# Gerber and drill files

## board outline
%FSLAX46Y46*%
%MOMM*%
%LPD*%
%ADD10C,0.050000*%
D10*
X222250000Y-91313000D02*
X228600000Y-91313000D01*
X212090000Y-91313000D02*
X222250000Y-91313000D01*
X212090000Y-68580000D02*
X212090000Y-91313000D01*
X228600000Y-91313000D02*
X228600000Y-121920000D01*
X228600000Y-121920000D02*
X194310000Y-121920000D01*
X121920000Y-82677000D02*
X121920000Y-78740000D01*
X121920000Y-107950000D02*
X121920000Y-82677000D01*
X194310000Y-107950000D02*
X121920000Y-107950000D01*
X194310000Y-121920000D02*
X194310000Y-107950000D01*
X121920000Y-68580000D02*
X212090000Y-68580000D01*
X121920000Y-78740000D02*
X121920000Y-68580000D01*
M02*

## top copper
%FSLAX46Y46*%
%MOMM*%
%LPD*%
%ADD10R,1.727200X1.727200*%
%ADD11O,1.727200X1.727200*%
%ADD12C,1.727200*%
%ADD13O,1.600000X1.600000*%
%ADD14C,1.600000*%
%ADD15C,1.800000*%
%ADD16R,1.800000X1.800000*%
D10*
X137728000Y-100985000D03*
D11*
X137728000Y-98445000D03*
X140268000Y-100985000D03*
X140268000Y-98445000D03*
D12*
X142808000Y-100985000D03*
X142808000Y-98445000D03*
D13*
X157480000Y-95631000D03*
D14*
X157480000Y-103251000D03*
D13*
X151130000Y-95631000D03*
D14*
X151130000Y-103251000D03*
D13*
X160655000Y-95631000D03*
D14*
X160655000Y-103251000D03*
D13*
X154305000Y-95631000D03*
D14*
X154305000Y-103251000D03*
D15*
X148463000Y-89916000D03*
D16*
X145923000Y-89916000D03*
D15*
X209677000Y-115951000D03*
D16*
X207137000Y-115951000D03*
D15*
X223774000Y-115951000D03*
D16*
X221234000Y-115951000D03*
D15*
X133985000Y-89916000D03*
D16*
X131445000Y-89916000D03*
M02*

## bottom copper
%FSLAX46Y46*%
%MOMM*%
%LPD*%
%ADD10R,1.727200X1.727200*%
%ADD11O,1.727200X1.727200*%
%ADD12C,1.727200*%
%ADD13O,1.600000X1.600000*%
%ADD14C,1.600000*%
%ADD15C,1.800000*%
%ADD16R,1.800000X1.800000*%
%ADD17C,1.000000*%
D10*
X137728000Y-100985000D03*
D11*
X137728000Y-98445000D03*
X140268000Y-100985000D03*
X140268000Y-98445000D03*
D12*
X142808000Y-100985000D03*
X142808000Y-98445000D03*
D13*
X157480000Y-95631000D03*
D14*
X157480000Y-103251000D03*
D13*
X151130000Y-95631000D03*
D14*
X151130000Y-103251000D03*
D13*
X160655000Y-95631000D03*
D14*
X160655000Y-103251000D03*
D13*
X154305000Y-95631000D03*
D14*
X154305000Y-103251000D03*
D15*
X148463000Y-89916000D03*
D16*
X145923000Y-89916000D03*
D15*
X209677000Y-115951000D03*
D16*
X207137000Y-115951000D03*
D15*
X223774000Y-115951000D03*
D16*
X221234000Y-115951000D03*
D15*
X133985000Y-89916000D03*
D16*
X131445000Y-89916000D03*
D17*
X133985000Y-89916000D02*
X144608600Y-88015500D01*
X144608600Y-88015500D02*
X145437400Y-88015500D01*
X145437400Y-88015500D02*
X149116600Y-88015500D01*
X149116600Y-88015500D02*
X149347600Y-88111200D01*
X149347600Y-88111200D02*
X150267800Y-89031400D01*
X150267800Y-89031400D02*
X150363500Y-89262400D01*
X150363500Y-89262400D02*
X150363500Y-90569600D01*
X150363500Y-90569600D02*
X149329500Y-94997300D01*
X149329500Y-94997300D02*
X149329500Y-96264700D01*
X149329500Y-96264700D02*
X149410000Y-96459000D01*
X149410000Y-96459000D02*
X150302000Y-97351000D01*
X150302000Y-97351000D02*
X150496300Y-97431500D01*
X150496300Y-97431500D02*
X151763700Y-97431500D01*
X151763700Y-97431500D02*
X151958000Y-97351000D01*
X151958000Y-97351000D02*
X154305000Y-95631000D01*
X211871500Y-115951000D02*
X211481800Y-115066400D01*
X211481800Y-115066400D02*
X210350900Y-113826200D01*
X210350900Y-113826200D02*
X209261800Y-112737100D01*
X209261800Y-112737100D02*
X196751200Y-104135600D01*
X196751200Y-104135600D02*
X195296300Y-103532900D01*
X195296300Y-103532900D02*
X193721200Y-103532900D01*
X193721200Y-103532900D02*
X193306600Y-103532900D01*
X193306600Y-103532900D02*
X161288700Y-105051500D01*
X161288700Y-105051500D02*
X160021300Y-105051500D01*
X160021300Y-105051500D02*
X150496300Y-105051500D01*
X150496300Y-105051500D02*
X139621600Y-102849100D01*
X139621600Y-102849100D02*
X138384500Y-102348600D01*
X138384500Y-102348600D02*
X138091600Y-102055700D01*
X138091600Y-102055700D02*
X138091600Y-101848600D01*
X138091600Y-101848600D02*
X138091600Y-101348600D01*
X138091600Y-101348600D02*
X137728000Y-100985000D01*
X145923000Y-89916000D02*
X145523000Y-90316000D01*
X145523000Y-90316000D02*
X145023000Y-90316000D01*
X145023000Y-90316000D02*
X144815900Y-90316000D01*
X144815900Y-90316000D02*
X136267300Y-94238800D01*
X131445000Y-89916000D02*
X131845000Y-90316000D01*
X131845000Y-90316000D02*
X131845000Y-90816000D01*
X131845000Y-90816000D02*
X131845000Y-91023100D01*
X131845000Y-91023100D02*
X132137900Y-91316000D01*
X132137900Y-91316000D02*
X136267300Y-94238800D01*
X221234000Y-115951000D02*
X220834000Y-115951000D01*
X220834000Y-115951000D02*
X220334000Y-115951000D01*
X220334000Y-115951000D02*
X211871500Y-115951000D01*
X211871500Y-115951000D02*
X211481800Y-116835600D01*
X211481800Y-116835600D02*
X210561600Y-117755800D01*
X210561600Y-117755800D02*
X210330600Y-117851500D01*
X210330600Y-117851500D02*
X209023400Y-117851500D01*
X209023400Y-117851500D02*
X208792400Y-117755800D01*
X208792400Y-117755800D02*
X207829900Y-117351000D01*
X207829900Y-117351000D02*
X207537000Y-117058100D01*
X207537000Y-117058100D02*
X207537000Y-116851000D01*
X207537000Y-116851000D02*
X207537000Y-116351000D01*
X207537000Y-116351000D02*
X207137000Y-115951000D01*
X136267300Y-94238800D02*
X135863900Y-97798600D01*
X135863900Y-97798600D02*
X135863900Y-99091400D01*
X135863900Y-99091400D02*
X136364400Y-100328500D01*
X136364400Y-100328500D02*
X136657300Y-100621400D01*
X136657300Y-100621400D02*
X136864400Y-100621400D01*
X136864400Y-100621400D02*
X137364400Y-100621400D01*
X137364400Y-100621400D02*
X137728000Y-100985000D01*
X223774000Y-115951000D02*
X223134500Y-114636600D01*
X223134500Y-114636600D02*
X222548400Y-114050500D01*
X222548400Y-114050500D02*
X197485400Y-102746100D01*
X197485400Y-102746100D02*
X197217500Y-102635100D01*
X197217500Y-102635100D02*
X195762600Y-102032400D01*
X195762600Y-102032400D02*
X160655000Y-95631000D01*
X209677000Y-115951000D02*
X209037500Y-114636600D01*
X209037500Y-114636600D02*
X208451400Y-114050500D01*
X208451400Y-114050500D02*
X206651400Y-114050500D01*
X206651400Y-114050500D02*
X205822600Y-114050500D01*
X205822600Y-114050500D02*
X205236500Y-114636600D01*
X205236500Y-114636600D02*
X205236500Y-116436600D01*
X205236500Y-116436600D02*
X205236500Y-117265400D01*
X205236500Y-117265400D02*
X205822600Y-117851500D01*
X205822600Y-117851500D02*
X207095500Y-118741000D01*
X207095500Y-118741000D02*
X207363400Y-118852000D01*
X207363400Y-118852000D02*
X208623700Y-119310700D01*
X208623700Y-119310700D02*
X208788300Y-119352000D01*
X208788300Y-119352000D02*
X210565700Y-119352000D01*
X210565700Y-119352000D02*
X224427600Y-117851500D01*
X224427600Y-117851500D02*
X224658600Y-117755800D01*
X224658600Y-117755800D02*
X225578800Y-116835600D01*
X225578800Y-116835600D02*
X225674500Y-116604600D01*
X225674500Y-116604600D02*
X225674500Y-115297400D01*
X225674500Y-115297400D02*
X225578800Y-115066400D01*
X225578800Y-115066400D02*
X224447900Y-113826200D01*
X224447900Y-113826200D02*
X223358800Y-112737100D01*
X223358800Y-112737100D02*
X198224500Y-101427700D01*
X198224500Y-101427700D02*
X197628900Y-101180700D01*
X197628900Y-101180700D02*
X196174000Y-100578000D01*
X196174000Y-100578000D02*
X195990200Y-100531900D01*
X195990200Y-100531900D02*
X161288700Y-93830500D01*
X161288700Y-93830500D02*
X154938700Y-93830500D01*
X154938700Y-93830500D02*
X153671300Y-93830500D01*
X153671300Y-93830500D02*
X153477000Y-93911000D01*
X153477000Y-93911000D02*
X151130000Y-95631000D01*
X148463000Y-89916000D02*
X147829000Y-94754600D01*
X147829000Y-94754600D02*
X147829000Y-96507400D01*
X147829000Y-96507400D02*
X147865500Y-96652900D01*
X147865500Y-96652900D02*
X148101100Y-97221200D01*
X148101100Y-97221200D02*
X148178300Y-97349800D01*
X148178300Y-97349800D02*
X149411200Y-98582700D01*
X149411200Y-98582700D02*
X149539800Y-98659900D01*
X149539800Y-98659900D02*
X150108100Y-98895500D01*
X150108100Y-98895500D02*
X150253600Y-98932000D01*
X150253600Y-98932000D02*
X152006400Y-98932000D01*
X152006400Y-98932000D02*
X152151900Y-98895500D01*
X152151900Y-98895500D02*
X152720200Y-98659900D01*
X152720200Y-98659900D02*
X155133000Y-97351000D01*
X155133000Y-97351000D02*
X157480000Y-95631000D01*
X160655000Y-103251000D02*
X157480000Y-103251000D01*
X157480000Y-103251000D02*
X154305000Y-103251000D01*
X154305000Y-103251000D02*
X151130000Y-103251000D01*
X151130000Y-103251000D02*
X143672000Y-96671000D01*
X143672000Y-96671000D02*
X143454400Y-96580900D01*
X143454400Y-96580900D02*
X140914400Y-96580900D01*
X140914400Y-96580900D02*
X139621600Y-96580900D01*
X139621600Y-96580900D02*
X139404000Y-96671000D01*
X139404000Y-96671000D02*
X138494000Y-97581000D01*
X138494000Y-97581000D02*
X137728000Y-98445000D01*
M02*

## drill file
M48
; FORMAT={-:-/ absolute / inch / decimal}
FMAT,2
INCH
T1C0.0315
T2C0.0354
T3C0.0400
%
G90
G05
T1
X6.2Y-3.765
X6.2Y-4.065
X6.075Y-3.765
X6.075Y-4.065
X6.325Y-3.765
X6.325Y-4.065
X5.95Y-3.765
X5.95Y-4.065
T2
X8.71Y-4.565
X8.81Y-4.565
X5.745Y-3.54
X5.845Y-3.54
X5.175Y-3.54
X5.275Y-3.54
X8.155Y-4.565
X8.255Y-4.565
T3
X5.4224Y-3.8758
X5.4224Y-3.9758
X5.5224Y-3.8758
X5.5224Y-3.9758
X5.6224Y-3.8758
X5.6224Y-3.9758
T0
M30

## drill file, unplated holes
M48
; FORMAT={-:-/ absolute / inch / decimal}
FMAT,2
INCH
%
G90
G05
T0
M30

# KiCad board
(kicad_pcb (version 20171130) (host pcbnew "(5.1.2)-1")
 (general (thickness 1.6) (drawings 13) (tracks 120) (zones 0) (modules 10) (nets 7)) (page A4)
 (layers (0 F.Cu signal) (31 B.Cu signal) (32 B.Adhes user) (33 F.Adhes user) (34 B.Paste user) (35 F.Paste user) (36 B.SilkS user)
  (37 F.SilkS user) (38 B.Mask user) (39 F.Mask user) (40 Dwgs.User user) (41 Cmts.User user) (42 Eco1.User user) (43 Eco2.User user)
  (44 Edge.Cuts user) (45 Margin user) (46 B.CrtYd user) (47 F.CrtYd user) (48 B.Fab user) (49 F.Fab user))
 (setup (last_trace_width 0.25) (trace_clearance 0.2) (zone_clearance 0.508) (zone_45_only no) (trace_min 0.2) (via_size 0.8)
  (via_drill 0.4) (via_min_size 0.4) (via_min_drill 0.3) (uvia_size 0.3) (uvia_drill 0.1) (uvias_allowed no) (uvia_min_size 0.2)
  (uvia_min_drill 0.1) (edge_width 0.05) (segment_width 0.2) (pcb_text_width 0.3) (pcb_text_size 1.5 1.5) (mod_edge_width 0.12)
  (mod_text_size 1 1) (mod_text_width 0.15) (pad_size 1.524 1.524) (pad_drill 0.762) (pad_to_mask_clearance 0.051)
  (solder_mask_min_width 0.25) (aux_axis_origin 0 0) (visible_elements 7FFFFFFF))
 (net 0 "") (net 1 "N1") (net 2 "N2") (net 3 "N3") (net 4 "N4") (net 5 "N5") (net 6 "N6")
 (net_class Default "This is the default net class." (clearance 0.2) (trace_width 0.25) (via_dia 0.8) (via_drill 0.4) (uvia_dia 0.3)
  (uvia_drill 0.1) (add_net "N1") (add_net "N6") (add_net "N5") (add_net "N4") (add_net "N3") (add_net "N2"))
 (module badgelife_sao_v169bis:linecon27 (layer F.Cu) (at 173.482 93.345)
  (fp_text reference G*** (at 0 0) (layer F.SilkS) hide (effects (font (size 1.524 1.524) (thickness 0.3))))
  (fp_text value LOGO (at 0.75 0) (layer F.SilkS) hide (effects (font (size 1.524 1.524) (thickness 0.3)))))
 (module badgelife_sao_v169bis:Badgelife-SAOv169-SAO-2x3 (layer F.Cu) (at 140.208 99.695)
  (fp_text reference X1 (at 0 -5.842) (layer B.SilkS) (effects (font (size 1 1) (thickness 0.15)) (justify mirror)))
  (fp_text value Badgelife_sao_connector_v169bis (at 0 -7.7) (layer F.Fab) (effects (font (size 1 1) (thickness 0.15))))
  (pad 2 thru_hole rect (at -2.48 1.29 270) (size 1.7272 1.7272) (drill 1.016) (layers *.Cu *.Mask) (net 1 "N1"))
  (pad 1 thru_hole oval (at -2.48 -1.25 270) (size 1.7272 1.7272) (drill 1.016) (layers *.Cu *.Mask) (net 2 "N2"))
  (pad 4 thru_hole oval (at 0.06 1.29 270) (size 1.7272 1.7272) (drill 1.016) (layers *.Cu *.Mask))
  (pad 3 thru_hole oval (at 0.06 -1.25 270) (size 1.7272 1.7272) (drill 1.016) (layers *.Cu *.Mask))
  (pad 6 thru_hole circle (at 2.6 1.29 270) (size 1.7272 1.7272) (drill 1.016) (layers *.Cu *.Mask))
  (pad 5 thru_hole circle (at 2.6 -1.25 270) (size 1.7272 1.7272) (drill 1.016) (layers *.Cu *.Mask)))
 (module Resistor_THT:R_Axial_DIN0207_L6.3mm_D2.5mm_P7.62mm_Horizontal (layer F.Cu) (at 157.48 103.251 90)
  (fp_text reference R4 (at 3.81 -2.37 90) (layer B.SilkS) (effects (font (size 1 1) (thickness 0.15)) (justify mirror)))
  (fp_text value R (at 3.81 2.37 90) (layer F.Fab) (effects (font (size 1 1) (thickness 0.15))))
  (pad 2 thru_hole oval (at 7.62 0 90) (size 1.6 1.6) (drill 0.8) (layers *.Cu *.Mask) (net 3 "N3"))
  (pad 1 thru_hole circle (at 0 0 90) (size 1.6 1.6) (drill 0.8) (layers *.Cu *.Mask) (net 2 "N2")))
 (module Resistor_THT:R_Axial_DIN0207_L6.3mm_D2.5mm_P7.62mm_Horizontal (layer F.Cu) (at 151.13 103.251 90)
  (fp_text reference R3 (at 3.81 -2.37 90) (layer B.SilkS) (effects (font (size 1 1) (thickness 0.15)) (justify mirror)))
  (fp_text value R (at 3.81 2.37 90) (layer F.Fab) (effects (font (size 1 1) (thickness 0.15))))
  (pad 2 thru_hole oval (at 7.62 0 90) (size 1.6 1.6) (drill 0.8) (layers *.Cu *.Mask) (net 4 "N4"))
  (pad 1 thru_hole circle (at 0 0 90) (size 1.6 1.6) (drill 0.8) (layers *.Cu *.Mask) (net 2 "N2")))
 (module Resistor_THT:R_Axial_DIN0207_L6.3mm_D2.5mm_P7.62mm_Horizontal (layer F.Cu) (at 160.655 103.251 90)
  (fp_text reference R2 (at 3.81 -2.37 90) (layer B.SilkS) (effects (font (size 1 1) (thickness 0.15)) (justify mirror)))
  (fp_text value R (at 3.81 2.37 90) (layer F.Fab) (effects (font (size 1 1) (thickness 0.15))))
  (pad 2 thru_hole oval (at 7.62 0 90) (size 1.6 1.6) (drill 0.8) (layers *.Cu *.Mask) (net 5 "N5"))
  (pad 1 thru_hole circle (at 0 0 90) (size 1.6 1.6) (drill 0.8) (layers *.Cu *.Mask) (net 2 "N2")))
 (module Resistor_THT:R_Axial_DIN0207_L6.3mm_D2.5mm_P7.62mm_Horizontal (layer F.Cu) (at 154.305 103.251 90)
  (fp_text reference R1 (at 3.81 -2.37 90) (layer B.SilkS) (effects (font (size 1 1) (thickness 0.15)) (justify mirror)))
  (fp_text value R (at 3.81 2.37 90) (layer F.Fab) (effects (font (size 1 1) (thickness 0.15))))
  (pad 2 thru_hole oval (at 7.62 0 90) (size 1.6 1.6) (drill 0.8) (layers *.Cu *.Mask) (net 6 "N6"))
  (pad 1 thru_hole circle (at 0 0 90) (size 1.6 1.6) (drill 0.8) (layers *.Cu *.Mask) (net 2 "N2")))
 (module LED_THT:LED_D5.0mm (layer F.Cu) (at 145.923 89.916)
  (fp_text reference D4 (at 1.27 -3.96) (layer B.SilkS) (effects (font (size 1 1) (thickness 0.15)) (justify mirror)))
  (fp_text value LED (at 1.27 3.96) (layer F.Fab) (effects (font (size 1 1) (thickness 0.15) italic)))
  (pad 2 thru_hole circle (at 2.54 0) (size 1.8 1.8) (drill 0.9) (layers *.Cu *.Mask) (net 3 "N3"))
  (pad 1 thru_hole rect (at 0 0) (size 1.8 1.8) (drill 0.9) (layers *.Cu *.Mask) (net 1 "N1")))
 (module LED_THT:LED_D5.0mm (layer F.Cu) (at 207.137 115.951)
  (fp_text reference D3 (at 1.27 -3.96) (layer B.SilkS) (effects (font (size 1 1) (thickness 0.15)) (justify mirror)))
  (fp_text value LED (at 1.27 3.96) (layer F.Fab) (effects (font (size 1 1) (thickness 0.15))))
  (pad 2 thru_hole circle (at 2.54 0) (size 1.8 1.8) (drill 0.9) (layers *.Cu *.Mask) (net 4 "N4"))
  (pad 1 thru_hole rect (at 0 0) (size 1.8 1.8) (drill 0.9) (layers *.Cu *.Mask) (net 1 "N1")))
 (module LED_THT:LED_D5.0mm (layer F.Cu) (at 221.234 115.951)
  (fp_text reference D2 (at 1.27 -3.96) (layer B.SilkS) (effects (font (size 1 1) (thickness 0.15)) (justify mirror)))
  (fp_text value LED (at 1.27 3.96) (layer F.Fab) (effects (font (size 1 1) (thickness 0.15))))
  (pad 2 thru_hole circle (at 2.54 0) (size 1.8 1.8) (drill 0.9) (layers *.Cu *.Mask) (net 5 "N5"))
  (pad 1 thru_hole rect (at 0 0) (size 1.8 1.8) (drill 0.9) (layers *.Cu *.Mask) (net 1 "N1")))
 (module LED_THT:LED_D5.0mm (layer F.Cu) (at 131.445 89.916)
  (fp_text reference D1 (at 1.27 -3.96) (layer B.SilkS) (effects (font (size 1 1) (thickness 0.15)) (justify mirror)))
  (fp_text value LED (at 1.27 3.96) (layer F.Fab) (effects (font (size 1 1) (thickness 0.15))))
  (pad 2 thru_hole circle (at 2.54 0) (size 1.8 1.8) (drill 0.9) (layers *.Cu *.Mask) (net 6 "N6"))
  (pad 1 thru_hole rect (at 0 0) (size 1.8 1.8) (drill 0.9) (layers *.Cu *.Mask) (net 1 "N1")))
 (gr_line (start 222.25 91.313) (end 228.6 91.313) (layer Edge.Cuts) (width 0.05))
 (gr_line (start 212.09 91.313) (end 222.25 91.313) (layer Edge.Cuts) (width 0.05))
 (gr_line (start 212.09 68.58) (end 212.09 91.313) (layer Edge.Cuts) (width 0.05))
 (gr_line (start 228.6 91.313) (end 228.6 121.92) (layer Edge.Cuts) (width 0.05))
 (gr_line (start 228.6 121.92) (end 194.31 121.92) (layer Edge.Cuts) (width 0.05))
 (gr_line (start 121.92 82.677) (end 121.92 78.74) (layer Edge.Cuts) (width 0.05))
 (gr_line (start 121.92 107.95) (end 121.92 82.677) (layer Edge.Cuts) (width 0.05))
 (gr_line (start 194.31 107.95) (end 121.92 107.95) (layer Edge.Cuts) (width 0.05))
 (gr_line (start 194.31 121.92) (end 194.31 107.95) (layer Edge.Cuts) (width 0.05))
 (gr_line (start 121.92 68.58) (end 212.09 68.58) (layer Edge.Cuts) (width 0.05))
 (gr_line (start 121.92 78.74) (end 121.92 68.58) (layer Edge.Cuts) (width 0.05))
 (segment (start 133.985 89.916) (end 144.6086 88.0155) (width 1) (layer B.Cu) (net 6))
 (segment (start 144.6086 88.0155) (end 145.4374 88.0155) (width 1) (layer B.Cu) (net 6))
 (segment (start 145.4374 88.0155) (end 149.1166 88.0155) (width 1) (layer B.Cu) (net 6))
 (segment (start 149.1166 88.0155) (end 149.3476 88.1112) (width 1) (layer B.Cu) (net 6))
 (segment (start 149.3476 88.1112) (end 150.2678 89.0314) (width 1) (layer B.Cu) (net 6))
 (segment (start 150.2678 89.0314) (end 150.3635 89.2624) (width 1) (layer B.Cu) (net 6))
 (segment (start 150.3635 89.2624) (end 150.3635 90.5696) (width 1) (layer B.Cu) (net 6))
 (segment (start 150.3635 90.5696) (end 149.3295 94.9973) (width 1) (layer B.Cu) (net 6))
 (segment (start 149.3295 94.9973) (end 149.3295 96.2647) (width 1) (layer B.Cu) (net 6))
 (segment (start 149.3295 96.2647) (end 149.41 96.459) (width 1) (layer B.Cu) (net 6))
 (segment (start 149.41 96.459) (end 150.302 97.351) (width 1) (layer B.Cu) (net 6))
 (segment (start 150.302 97.351) (end 150.4963 97.4315) (width 1) (layer B.Cu) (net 6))
 (segment (start 150.4963 97.4315) (end 151.7637 97.4315) (width 1) (layer B.Cu) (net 6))
 (segment (start 151.7637 97.4315) (end 151.958 97.351) (width 1) (layer B.Cu) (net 6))
 (segment (start 151.958 97.351) (end 154.305 95.631) (width 1) (layer B.Cu) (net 6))
 (segment (start 211.8715 115.951) (end 211.4818 115.0664) (width 1) (layer B.Cu) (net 1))
 (segment (start 211.4818 115.0664) (end 210.3509 113.8262) (width 1) (layer B.Cu) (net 1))
 (segment (start 210.3509 113.8262) (end 209.2618 112.7371) (width 1) (layer B.Cu) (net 1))
 (segment (start 209.2618 112.7371) (end 196.7512 104.1356) (width 1) (layer B.Cu) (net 1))
 (segment (start 196.7512 104.1356) (end 195.2963 103.5329) (width 1) (layer B.Cu) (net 1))
 (segment (start 195.2963 103.5329) (end 193.7212 103.5329) (width 1) (layer B.Cu) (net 1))
 (segment (start 193.7212 103.5329) (end 193.3066 103.5329) (width 1) (layer B.Cu) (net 1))
 (segment (start 193.3066 103.5329) (end 161.2887 105.0515) (width 1) (layer B.Cu) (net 1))
 (segment (start 161.2887 105.0515) (end 160.0213 105.0515) (width 1) (layer B.Cu) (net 1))
 (segment (start 160.0213 105.0515) (end 150.4963 105.0515) (width 1) (layer B.Cu) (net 1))
 (segment (start 150.4963 105.0515) (end 139.6216 102.8491) (width 1) (layer B.Cu) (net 1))
 (segment (start 139.6216 102.8491) (end 138.3845 102.3486) (width 1) (layer B.Cu) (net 1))
 (segment (start 138.3845 102.3486) (end 138.0916 102.0557) (width 1) (layer B.Cu) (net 1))
 (segment (start 138.0916 102.0557) (end 138.0916 101.8486) (width 1) (layer B.Cu) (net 1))
 (segment (start 138.0916 101.8486) (end 138.0916 101.3486) (width 1) (layer B.Cu) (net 1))
 (segment (start 138.0916 101.3486) (end 137.728 100.985) (width 1) (layer B.Cu) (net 1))
 (segment (start 145.923 89.916) (end 145.523 90.316) (width 1) (layer B.Cu) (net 1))
 (segment (start 145.523 90.316) (end 145.023 90.316) (width 1) (layer B.Cu) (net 1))
 (segment (start 145.023 90.316) (end 144.8159 90.316) (width 1) (layer B.Cu) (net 1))
 (segment (start 144.8159 90.316) (end 136.2673 94.2388) (width 1) (layer B.Cu) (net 1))
 (segment (start 131.445 89.916) (end 131.845 90.316) (width 1) (layer B.Cu) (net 1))
 (segment (start 131.845 90.316) (end 131.845 90.816) (width 1) (layer B.Cu) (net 1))
 (segment (start 131.845 90.816) (end 131.845 91.0231) (width 1) (layer B.Cu) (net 1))
 (segment (start 131.845 91.0231) (end 132.1379 91.316) (width 1) (layer B.Cu) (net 1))
 (segment (start 132.1379 91.316) (end 136.2673 94.2388) (width 1) (layer B.Cu) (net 1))
 (segment (start 221.234 115.951) (end 220.834 115.951) (width 1) (layer B.Cu) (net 1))
 (segment (start 220.834 115.951) (end 220.334 115.951) (width 1) (layer B.Cu) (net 1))
 (segment (start 220.334 115.951) (end 211.8715 115.951) (width 1) (layer B.Cu) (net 1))
 (segment (start 211.8715 115.951) (end 211.4818 116.8356) (width 1) (layer B.Cu) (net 1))
 (segment (start 211.4818 116.8356) (end 210.5616 117.7558) (width 1) (layer B.Cu) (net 1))
 (segment (start 210.5616 117.7558) (end 210.3306 117.8515) (width 1) (layer B.Cu) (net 1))
 (segment (start 210.3306 117.8515) (end 209.0234 117.8515) (width 1) (layer B.Cu) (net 1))
 (segment (start 209.0234 117.8515) (end 208.7924 117.7558) (width 1) (layer B.Cu) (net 1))
 (segment (start 208.7924 117.7558) (end 207.8299 117.351) (width 1) (layer B.Cu) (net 1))
 (segment (start 207.8299 117.351) (end 207.537 117.0581) (width 1) (layer B.Cu) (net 1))
 (segment (start 207.537 117.0581) (end 207.537 116.851) (width 1) (layer B.Cu) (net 1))
 (segment (start 207.537 116.851) (end 207.537 116.351) (width 1) (layer B.Cu) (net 1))
 (segment (start 207.537 116.351) (end 207.137 115.951) (width 1) (layer B.Cu) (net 1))
 (segment (start 136.2673 94.2388) (end 135.8639 97.7986) (width 1) (layer B.Cu) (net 1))
 (segment (start 135.8639 97.7986) (end 135.8639 99.0914) (width 1) (layer B.Cu) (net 1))
 (segment (start 135.8639 99.0914) (end 136.3644 100.3285) (width 1) (layer B.Cu) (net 1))
 (segment (start 136.3644 100.3285) (end 136.6573 100.6214) (width 1) (layer B.Cu) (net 1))
 (segment (start 136.6573 100.6214) (end 136.8644 100.6214) (width 1) (layer B.Cu) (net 1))
 (segment (start 136.8644 100.6214) (end 137.3644 100.6214) (width 1) (layer B.Cu) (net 1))
 (segment (start 137.3644 100.6214) (end 137.728 100.985) (width 1) (layer B.Cu) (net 1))
 (segment (start 223.774 115.951) (end 223.1345 114.6366) (width 1) (layer B.Cu) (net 5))
 (segment (start 223.1345 114.6366) (end 222.5484 114.0505) (width 1) (layer B.Cu) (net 5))
 (segment (start 222.5484 114.0505) (end 197.4854 102.7461) (width 1) (layer B.Cu) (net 5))
 (segment (start 197.4854 102.7461) (end 197.2175 102.6351) (width 1) (layer B.Cu) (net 5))
 (segment (start 197.2175 102.6351) (end 195.7626 102.0324) (width 1) (layer B.Cu) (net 5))
 (segment (start 195.7626 102.0324) (end 160.655 95.631) (width 1) (layer B.Cu) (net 5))
 (segment (start 209.677 115.951) (end 209.0375 114.6366) (width 1) (layer B.Cu) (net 4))
 (segment (start 209.0375 114.6366) (end 208.4514 114.0505) (width 1) (layer B.Cu) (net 4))
 (segment (start 208.4514 114.0505) (end 206.6514 114.0505) (width 1) (layer B.Cu) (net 4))
 (segment (start 206.6514 114.0505) (end 205.8226 114.0505) (width 1) (layer B.Cu) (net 4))
 (segment (start 205.8226 114.0505) (end 205.2365 114.6366) (width 1) (layer B.Cu) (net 4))
 (segment (start 205.2365 114.6366) (end 205.2365 116.4366) (width 1) (layer B.Cu) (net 4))
 (segment (start 205.2365 116.4366) (end 205.2365 117.2654) (width 1) (layer B.Cu) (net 4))
 (segment (start 205.2365 117.2654) (end 205.8226 117.8515) (width 1) (layer B.Cu) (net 4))
 (segment (start 205.8226 117.8515) (end 207.0955 118.741) (width 1) (layer B.Cu) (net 4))
 (segment (start 207.0955 118.741) (end 207.3634 118.852) (width 1) (layer B.Cu) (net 4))
 (segment (start 207.3634 118.852) (end 208.6237 119.3107) (width 1) (layer B.Cu) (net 4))
 (segment (start 208.6237 119.3107) (end 208.7883 119.352) (width 1) (layer B.Cu) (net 4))
 (segment (start 208.7883 119.352) (end 210.5657 119.352) (width 1) (layer B.Cu) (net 4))
 (segment (start 210.5657 119.352) (end 224.4276 117.8515) (width 1) (layer B.Cu) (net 4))
 (segment (start 224.4276 117.8515) (end 224.6586 117.7558) (width 1) (layer B.Cu) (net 4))
 (segment (start 224.6586 117.7558) (end 225.5788 116.8356) (width 1) (layer B.Cu) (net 4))
 (segment (start 225.5788 116.8356) (end 225.6745 116.6046) (width 1) (layer B.Cu) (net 4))
 (segment (start 225.6745 116.6046) (end 225.6745 115.2974) (width 1) (layer B.Cu) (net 4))
 (segment (start 225.6745 115.2974) (end 225.5788 115.0664) (width 1) (layer B.Cu) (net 4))
 (segment (start 225.5788 115.0664) (end 224.4479 113.8262) (width 1) (layer B.Cu) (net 4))
 (segment (start 224.4479 113.8262) (end 223.3588 112.7371) (width 1) (layer B.Cu) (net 4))
 (segment (start 223.3588 112.7371) (end 198.2245 101.4277) (width 1) (layer B.Cu) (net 4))
 (segment (start 198.2245 101.4277) (end 197.6289 101.1807) (width 1) (layer B.Cu) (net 4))
 (segment (start 197.6289 101.1807) (end 196.174 100.578) (width 1) (layer B.Cu) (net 4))
 (segment (start 196.174 100.578) (end 195.9902 100.5319) (width 1) (layer B.Cu) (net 4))
 (segment (start 195.9902 100.5319) (end 161.2887 93.8305) (width 1) (layer B.Cu) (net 4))
 (segment (start 161.2887 93.8305) (end 154.9387 93.8305) (width 1) (layer B.Cu) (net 4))
 (segment (start 154.9387 93.8305) (end 153.6713 93.8305) (width 1) (layer B.Cu) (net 4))
 (segment (start 153.6713 93.8305) (end 153.477 93.911) (width 1) (layer B.Cu) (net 4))
 (segment (start 153.477 93.911) (end 151.13 95.631) (width 1) (layer B.Cu) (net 4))
 (segment (start 148.463 89.916) (end 147.829 94.7546) (width 1) (layer B.Cu) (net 3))
 (segment (start 147.829 94.7546) (end 147.829 96.5074) (width 1) (layer B.Cu) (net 3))
 (segment (start 147.829 96.5074) (end 147.8655 96.6529) (width 1) (layer B.Cu) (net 3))
 (segment (start 147.8655 96.6529) (end 148.1011 97.2212) (width 1) (layer B.Cu) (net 3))
 (segment (start 148.1011 97.2212) (end 148.1783 97.3498) (width 1) (layer B.Cu) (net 3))
 (segment (start 148.1783 97.3498) (end 149.4112 98.5827) (width 1) (layer B.Cu) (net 3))
 (segment (start 149.4112 98.5827) (end 149.5398 98.6599) (width 1) (layer B.Cu) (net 3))
 (segment (start 149.5398 98.6599) (end 150.1081 98.8955) (width 1) (layer B.Cu) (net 3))
 (segment (start 150.1081 98.8955) (end 150.2536 98.932) (width 1) (layer B.Cu) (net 3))
 (segment (start 150.2536 98.932) (end 152.0064 98.932) (width 1) (layer B.Cu) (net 3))
 (segment (start 152.0064 98.932) (end 152.1519 98.8955) (width 1) (layer B.Cu) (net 3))
 (segment (start 152.1519 98.8955) (end 152.7202 98.6599) (width 1) (layer B.Cu) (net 3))
 (segment (start 152.7202 98.6599) (end 155.133 97.351) (width 1) (layer B.Cu) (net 3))
 (segment (start 155.133 97.351) (end 157.48 95.631) (width 1) (layer B.Cu) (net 3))
 (segment (start 160.655 103.251) (end 157.48 103.251) (width 1) (layer B.Cu) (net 2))
 (segment (start 157.48 103.251) (end 154.305 103.251) (width 1) (layer B.Cu) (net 2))
 (segment (start 154.305 103.251) (end 151.13 103.251) (width 1) (layer B.Cu) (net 2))
 (segment (start 151.13 103.251) (end 143.672 96.671) (width 1) (layer B.Cu) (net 2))
 (segment (start 143.672 96.671) (end 143.4544 96.5809) (width 1) (layer B.Cu) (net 2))
 (segment (start 143.4544 96.5809) (end 140.9144 96.5809) (width 1) (layer B.Cu) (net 2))
 (segment (start 140.9144 96.5809) (end 139.6216 96.5809) (width 1) (layer B.Cu) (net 2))
 (segment (start 139.6216 96.5809) (end 139.404 96.671) (width 1) (layer B.Cu) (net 2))
 (segment (start 139.404 96.671) (end 138.494 97.581) (width 1) (layer B.Cu) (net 2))
 (segment (start 138.494 97.581) (end 137.728 98.445) (width 1) (layer B.Cu) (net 2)))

